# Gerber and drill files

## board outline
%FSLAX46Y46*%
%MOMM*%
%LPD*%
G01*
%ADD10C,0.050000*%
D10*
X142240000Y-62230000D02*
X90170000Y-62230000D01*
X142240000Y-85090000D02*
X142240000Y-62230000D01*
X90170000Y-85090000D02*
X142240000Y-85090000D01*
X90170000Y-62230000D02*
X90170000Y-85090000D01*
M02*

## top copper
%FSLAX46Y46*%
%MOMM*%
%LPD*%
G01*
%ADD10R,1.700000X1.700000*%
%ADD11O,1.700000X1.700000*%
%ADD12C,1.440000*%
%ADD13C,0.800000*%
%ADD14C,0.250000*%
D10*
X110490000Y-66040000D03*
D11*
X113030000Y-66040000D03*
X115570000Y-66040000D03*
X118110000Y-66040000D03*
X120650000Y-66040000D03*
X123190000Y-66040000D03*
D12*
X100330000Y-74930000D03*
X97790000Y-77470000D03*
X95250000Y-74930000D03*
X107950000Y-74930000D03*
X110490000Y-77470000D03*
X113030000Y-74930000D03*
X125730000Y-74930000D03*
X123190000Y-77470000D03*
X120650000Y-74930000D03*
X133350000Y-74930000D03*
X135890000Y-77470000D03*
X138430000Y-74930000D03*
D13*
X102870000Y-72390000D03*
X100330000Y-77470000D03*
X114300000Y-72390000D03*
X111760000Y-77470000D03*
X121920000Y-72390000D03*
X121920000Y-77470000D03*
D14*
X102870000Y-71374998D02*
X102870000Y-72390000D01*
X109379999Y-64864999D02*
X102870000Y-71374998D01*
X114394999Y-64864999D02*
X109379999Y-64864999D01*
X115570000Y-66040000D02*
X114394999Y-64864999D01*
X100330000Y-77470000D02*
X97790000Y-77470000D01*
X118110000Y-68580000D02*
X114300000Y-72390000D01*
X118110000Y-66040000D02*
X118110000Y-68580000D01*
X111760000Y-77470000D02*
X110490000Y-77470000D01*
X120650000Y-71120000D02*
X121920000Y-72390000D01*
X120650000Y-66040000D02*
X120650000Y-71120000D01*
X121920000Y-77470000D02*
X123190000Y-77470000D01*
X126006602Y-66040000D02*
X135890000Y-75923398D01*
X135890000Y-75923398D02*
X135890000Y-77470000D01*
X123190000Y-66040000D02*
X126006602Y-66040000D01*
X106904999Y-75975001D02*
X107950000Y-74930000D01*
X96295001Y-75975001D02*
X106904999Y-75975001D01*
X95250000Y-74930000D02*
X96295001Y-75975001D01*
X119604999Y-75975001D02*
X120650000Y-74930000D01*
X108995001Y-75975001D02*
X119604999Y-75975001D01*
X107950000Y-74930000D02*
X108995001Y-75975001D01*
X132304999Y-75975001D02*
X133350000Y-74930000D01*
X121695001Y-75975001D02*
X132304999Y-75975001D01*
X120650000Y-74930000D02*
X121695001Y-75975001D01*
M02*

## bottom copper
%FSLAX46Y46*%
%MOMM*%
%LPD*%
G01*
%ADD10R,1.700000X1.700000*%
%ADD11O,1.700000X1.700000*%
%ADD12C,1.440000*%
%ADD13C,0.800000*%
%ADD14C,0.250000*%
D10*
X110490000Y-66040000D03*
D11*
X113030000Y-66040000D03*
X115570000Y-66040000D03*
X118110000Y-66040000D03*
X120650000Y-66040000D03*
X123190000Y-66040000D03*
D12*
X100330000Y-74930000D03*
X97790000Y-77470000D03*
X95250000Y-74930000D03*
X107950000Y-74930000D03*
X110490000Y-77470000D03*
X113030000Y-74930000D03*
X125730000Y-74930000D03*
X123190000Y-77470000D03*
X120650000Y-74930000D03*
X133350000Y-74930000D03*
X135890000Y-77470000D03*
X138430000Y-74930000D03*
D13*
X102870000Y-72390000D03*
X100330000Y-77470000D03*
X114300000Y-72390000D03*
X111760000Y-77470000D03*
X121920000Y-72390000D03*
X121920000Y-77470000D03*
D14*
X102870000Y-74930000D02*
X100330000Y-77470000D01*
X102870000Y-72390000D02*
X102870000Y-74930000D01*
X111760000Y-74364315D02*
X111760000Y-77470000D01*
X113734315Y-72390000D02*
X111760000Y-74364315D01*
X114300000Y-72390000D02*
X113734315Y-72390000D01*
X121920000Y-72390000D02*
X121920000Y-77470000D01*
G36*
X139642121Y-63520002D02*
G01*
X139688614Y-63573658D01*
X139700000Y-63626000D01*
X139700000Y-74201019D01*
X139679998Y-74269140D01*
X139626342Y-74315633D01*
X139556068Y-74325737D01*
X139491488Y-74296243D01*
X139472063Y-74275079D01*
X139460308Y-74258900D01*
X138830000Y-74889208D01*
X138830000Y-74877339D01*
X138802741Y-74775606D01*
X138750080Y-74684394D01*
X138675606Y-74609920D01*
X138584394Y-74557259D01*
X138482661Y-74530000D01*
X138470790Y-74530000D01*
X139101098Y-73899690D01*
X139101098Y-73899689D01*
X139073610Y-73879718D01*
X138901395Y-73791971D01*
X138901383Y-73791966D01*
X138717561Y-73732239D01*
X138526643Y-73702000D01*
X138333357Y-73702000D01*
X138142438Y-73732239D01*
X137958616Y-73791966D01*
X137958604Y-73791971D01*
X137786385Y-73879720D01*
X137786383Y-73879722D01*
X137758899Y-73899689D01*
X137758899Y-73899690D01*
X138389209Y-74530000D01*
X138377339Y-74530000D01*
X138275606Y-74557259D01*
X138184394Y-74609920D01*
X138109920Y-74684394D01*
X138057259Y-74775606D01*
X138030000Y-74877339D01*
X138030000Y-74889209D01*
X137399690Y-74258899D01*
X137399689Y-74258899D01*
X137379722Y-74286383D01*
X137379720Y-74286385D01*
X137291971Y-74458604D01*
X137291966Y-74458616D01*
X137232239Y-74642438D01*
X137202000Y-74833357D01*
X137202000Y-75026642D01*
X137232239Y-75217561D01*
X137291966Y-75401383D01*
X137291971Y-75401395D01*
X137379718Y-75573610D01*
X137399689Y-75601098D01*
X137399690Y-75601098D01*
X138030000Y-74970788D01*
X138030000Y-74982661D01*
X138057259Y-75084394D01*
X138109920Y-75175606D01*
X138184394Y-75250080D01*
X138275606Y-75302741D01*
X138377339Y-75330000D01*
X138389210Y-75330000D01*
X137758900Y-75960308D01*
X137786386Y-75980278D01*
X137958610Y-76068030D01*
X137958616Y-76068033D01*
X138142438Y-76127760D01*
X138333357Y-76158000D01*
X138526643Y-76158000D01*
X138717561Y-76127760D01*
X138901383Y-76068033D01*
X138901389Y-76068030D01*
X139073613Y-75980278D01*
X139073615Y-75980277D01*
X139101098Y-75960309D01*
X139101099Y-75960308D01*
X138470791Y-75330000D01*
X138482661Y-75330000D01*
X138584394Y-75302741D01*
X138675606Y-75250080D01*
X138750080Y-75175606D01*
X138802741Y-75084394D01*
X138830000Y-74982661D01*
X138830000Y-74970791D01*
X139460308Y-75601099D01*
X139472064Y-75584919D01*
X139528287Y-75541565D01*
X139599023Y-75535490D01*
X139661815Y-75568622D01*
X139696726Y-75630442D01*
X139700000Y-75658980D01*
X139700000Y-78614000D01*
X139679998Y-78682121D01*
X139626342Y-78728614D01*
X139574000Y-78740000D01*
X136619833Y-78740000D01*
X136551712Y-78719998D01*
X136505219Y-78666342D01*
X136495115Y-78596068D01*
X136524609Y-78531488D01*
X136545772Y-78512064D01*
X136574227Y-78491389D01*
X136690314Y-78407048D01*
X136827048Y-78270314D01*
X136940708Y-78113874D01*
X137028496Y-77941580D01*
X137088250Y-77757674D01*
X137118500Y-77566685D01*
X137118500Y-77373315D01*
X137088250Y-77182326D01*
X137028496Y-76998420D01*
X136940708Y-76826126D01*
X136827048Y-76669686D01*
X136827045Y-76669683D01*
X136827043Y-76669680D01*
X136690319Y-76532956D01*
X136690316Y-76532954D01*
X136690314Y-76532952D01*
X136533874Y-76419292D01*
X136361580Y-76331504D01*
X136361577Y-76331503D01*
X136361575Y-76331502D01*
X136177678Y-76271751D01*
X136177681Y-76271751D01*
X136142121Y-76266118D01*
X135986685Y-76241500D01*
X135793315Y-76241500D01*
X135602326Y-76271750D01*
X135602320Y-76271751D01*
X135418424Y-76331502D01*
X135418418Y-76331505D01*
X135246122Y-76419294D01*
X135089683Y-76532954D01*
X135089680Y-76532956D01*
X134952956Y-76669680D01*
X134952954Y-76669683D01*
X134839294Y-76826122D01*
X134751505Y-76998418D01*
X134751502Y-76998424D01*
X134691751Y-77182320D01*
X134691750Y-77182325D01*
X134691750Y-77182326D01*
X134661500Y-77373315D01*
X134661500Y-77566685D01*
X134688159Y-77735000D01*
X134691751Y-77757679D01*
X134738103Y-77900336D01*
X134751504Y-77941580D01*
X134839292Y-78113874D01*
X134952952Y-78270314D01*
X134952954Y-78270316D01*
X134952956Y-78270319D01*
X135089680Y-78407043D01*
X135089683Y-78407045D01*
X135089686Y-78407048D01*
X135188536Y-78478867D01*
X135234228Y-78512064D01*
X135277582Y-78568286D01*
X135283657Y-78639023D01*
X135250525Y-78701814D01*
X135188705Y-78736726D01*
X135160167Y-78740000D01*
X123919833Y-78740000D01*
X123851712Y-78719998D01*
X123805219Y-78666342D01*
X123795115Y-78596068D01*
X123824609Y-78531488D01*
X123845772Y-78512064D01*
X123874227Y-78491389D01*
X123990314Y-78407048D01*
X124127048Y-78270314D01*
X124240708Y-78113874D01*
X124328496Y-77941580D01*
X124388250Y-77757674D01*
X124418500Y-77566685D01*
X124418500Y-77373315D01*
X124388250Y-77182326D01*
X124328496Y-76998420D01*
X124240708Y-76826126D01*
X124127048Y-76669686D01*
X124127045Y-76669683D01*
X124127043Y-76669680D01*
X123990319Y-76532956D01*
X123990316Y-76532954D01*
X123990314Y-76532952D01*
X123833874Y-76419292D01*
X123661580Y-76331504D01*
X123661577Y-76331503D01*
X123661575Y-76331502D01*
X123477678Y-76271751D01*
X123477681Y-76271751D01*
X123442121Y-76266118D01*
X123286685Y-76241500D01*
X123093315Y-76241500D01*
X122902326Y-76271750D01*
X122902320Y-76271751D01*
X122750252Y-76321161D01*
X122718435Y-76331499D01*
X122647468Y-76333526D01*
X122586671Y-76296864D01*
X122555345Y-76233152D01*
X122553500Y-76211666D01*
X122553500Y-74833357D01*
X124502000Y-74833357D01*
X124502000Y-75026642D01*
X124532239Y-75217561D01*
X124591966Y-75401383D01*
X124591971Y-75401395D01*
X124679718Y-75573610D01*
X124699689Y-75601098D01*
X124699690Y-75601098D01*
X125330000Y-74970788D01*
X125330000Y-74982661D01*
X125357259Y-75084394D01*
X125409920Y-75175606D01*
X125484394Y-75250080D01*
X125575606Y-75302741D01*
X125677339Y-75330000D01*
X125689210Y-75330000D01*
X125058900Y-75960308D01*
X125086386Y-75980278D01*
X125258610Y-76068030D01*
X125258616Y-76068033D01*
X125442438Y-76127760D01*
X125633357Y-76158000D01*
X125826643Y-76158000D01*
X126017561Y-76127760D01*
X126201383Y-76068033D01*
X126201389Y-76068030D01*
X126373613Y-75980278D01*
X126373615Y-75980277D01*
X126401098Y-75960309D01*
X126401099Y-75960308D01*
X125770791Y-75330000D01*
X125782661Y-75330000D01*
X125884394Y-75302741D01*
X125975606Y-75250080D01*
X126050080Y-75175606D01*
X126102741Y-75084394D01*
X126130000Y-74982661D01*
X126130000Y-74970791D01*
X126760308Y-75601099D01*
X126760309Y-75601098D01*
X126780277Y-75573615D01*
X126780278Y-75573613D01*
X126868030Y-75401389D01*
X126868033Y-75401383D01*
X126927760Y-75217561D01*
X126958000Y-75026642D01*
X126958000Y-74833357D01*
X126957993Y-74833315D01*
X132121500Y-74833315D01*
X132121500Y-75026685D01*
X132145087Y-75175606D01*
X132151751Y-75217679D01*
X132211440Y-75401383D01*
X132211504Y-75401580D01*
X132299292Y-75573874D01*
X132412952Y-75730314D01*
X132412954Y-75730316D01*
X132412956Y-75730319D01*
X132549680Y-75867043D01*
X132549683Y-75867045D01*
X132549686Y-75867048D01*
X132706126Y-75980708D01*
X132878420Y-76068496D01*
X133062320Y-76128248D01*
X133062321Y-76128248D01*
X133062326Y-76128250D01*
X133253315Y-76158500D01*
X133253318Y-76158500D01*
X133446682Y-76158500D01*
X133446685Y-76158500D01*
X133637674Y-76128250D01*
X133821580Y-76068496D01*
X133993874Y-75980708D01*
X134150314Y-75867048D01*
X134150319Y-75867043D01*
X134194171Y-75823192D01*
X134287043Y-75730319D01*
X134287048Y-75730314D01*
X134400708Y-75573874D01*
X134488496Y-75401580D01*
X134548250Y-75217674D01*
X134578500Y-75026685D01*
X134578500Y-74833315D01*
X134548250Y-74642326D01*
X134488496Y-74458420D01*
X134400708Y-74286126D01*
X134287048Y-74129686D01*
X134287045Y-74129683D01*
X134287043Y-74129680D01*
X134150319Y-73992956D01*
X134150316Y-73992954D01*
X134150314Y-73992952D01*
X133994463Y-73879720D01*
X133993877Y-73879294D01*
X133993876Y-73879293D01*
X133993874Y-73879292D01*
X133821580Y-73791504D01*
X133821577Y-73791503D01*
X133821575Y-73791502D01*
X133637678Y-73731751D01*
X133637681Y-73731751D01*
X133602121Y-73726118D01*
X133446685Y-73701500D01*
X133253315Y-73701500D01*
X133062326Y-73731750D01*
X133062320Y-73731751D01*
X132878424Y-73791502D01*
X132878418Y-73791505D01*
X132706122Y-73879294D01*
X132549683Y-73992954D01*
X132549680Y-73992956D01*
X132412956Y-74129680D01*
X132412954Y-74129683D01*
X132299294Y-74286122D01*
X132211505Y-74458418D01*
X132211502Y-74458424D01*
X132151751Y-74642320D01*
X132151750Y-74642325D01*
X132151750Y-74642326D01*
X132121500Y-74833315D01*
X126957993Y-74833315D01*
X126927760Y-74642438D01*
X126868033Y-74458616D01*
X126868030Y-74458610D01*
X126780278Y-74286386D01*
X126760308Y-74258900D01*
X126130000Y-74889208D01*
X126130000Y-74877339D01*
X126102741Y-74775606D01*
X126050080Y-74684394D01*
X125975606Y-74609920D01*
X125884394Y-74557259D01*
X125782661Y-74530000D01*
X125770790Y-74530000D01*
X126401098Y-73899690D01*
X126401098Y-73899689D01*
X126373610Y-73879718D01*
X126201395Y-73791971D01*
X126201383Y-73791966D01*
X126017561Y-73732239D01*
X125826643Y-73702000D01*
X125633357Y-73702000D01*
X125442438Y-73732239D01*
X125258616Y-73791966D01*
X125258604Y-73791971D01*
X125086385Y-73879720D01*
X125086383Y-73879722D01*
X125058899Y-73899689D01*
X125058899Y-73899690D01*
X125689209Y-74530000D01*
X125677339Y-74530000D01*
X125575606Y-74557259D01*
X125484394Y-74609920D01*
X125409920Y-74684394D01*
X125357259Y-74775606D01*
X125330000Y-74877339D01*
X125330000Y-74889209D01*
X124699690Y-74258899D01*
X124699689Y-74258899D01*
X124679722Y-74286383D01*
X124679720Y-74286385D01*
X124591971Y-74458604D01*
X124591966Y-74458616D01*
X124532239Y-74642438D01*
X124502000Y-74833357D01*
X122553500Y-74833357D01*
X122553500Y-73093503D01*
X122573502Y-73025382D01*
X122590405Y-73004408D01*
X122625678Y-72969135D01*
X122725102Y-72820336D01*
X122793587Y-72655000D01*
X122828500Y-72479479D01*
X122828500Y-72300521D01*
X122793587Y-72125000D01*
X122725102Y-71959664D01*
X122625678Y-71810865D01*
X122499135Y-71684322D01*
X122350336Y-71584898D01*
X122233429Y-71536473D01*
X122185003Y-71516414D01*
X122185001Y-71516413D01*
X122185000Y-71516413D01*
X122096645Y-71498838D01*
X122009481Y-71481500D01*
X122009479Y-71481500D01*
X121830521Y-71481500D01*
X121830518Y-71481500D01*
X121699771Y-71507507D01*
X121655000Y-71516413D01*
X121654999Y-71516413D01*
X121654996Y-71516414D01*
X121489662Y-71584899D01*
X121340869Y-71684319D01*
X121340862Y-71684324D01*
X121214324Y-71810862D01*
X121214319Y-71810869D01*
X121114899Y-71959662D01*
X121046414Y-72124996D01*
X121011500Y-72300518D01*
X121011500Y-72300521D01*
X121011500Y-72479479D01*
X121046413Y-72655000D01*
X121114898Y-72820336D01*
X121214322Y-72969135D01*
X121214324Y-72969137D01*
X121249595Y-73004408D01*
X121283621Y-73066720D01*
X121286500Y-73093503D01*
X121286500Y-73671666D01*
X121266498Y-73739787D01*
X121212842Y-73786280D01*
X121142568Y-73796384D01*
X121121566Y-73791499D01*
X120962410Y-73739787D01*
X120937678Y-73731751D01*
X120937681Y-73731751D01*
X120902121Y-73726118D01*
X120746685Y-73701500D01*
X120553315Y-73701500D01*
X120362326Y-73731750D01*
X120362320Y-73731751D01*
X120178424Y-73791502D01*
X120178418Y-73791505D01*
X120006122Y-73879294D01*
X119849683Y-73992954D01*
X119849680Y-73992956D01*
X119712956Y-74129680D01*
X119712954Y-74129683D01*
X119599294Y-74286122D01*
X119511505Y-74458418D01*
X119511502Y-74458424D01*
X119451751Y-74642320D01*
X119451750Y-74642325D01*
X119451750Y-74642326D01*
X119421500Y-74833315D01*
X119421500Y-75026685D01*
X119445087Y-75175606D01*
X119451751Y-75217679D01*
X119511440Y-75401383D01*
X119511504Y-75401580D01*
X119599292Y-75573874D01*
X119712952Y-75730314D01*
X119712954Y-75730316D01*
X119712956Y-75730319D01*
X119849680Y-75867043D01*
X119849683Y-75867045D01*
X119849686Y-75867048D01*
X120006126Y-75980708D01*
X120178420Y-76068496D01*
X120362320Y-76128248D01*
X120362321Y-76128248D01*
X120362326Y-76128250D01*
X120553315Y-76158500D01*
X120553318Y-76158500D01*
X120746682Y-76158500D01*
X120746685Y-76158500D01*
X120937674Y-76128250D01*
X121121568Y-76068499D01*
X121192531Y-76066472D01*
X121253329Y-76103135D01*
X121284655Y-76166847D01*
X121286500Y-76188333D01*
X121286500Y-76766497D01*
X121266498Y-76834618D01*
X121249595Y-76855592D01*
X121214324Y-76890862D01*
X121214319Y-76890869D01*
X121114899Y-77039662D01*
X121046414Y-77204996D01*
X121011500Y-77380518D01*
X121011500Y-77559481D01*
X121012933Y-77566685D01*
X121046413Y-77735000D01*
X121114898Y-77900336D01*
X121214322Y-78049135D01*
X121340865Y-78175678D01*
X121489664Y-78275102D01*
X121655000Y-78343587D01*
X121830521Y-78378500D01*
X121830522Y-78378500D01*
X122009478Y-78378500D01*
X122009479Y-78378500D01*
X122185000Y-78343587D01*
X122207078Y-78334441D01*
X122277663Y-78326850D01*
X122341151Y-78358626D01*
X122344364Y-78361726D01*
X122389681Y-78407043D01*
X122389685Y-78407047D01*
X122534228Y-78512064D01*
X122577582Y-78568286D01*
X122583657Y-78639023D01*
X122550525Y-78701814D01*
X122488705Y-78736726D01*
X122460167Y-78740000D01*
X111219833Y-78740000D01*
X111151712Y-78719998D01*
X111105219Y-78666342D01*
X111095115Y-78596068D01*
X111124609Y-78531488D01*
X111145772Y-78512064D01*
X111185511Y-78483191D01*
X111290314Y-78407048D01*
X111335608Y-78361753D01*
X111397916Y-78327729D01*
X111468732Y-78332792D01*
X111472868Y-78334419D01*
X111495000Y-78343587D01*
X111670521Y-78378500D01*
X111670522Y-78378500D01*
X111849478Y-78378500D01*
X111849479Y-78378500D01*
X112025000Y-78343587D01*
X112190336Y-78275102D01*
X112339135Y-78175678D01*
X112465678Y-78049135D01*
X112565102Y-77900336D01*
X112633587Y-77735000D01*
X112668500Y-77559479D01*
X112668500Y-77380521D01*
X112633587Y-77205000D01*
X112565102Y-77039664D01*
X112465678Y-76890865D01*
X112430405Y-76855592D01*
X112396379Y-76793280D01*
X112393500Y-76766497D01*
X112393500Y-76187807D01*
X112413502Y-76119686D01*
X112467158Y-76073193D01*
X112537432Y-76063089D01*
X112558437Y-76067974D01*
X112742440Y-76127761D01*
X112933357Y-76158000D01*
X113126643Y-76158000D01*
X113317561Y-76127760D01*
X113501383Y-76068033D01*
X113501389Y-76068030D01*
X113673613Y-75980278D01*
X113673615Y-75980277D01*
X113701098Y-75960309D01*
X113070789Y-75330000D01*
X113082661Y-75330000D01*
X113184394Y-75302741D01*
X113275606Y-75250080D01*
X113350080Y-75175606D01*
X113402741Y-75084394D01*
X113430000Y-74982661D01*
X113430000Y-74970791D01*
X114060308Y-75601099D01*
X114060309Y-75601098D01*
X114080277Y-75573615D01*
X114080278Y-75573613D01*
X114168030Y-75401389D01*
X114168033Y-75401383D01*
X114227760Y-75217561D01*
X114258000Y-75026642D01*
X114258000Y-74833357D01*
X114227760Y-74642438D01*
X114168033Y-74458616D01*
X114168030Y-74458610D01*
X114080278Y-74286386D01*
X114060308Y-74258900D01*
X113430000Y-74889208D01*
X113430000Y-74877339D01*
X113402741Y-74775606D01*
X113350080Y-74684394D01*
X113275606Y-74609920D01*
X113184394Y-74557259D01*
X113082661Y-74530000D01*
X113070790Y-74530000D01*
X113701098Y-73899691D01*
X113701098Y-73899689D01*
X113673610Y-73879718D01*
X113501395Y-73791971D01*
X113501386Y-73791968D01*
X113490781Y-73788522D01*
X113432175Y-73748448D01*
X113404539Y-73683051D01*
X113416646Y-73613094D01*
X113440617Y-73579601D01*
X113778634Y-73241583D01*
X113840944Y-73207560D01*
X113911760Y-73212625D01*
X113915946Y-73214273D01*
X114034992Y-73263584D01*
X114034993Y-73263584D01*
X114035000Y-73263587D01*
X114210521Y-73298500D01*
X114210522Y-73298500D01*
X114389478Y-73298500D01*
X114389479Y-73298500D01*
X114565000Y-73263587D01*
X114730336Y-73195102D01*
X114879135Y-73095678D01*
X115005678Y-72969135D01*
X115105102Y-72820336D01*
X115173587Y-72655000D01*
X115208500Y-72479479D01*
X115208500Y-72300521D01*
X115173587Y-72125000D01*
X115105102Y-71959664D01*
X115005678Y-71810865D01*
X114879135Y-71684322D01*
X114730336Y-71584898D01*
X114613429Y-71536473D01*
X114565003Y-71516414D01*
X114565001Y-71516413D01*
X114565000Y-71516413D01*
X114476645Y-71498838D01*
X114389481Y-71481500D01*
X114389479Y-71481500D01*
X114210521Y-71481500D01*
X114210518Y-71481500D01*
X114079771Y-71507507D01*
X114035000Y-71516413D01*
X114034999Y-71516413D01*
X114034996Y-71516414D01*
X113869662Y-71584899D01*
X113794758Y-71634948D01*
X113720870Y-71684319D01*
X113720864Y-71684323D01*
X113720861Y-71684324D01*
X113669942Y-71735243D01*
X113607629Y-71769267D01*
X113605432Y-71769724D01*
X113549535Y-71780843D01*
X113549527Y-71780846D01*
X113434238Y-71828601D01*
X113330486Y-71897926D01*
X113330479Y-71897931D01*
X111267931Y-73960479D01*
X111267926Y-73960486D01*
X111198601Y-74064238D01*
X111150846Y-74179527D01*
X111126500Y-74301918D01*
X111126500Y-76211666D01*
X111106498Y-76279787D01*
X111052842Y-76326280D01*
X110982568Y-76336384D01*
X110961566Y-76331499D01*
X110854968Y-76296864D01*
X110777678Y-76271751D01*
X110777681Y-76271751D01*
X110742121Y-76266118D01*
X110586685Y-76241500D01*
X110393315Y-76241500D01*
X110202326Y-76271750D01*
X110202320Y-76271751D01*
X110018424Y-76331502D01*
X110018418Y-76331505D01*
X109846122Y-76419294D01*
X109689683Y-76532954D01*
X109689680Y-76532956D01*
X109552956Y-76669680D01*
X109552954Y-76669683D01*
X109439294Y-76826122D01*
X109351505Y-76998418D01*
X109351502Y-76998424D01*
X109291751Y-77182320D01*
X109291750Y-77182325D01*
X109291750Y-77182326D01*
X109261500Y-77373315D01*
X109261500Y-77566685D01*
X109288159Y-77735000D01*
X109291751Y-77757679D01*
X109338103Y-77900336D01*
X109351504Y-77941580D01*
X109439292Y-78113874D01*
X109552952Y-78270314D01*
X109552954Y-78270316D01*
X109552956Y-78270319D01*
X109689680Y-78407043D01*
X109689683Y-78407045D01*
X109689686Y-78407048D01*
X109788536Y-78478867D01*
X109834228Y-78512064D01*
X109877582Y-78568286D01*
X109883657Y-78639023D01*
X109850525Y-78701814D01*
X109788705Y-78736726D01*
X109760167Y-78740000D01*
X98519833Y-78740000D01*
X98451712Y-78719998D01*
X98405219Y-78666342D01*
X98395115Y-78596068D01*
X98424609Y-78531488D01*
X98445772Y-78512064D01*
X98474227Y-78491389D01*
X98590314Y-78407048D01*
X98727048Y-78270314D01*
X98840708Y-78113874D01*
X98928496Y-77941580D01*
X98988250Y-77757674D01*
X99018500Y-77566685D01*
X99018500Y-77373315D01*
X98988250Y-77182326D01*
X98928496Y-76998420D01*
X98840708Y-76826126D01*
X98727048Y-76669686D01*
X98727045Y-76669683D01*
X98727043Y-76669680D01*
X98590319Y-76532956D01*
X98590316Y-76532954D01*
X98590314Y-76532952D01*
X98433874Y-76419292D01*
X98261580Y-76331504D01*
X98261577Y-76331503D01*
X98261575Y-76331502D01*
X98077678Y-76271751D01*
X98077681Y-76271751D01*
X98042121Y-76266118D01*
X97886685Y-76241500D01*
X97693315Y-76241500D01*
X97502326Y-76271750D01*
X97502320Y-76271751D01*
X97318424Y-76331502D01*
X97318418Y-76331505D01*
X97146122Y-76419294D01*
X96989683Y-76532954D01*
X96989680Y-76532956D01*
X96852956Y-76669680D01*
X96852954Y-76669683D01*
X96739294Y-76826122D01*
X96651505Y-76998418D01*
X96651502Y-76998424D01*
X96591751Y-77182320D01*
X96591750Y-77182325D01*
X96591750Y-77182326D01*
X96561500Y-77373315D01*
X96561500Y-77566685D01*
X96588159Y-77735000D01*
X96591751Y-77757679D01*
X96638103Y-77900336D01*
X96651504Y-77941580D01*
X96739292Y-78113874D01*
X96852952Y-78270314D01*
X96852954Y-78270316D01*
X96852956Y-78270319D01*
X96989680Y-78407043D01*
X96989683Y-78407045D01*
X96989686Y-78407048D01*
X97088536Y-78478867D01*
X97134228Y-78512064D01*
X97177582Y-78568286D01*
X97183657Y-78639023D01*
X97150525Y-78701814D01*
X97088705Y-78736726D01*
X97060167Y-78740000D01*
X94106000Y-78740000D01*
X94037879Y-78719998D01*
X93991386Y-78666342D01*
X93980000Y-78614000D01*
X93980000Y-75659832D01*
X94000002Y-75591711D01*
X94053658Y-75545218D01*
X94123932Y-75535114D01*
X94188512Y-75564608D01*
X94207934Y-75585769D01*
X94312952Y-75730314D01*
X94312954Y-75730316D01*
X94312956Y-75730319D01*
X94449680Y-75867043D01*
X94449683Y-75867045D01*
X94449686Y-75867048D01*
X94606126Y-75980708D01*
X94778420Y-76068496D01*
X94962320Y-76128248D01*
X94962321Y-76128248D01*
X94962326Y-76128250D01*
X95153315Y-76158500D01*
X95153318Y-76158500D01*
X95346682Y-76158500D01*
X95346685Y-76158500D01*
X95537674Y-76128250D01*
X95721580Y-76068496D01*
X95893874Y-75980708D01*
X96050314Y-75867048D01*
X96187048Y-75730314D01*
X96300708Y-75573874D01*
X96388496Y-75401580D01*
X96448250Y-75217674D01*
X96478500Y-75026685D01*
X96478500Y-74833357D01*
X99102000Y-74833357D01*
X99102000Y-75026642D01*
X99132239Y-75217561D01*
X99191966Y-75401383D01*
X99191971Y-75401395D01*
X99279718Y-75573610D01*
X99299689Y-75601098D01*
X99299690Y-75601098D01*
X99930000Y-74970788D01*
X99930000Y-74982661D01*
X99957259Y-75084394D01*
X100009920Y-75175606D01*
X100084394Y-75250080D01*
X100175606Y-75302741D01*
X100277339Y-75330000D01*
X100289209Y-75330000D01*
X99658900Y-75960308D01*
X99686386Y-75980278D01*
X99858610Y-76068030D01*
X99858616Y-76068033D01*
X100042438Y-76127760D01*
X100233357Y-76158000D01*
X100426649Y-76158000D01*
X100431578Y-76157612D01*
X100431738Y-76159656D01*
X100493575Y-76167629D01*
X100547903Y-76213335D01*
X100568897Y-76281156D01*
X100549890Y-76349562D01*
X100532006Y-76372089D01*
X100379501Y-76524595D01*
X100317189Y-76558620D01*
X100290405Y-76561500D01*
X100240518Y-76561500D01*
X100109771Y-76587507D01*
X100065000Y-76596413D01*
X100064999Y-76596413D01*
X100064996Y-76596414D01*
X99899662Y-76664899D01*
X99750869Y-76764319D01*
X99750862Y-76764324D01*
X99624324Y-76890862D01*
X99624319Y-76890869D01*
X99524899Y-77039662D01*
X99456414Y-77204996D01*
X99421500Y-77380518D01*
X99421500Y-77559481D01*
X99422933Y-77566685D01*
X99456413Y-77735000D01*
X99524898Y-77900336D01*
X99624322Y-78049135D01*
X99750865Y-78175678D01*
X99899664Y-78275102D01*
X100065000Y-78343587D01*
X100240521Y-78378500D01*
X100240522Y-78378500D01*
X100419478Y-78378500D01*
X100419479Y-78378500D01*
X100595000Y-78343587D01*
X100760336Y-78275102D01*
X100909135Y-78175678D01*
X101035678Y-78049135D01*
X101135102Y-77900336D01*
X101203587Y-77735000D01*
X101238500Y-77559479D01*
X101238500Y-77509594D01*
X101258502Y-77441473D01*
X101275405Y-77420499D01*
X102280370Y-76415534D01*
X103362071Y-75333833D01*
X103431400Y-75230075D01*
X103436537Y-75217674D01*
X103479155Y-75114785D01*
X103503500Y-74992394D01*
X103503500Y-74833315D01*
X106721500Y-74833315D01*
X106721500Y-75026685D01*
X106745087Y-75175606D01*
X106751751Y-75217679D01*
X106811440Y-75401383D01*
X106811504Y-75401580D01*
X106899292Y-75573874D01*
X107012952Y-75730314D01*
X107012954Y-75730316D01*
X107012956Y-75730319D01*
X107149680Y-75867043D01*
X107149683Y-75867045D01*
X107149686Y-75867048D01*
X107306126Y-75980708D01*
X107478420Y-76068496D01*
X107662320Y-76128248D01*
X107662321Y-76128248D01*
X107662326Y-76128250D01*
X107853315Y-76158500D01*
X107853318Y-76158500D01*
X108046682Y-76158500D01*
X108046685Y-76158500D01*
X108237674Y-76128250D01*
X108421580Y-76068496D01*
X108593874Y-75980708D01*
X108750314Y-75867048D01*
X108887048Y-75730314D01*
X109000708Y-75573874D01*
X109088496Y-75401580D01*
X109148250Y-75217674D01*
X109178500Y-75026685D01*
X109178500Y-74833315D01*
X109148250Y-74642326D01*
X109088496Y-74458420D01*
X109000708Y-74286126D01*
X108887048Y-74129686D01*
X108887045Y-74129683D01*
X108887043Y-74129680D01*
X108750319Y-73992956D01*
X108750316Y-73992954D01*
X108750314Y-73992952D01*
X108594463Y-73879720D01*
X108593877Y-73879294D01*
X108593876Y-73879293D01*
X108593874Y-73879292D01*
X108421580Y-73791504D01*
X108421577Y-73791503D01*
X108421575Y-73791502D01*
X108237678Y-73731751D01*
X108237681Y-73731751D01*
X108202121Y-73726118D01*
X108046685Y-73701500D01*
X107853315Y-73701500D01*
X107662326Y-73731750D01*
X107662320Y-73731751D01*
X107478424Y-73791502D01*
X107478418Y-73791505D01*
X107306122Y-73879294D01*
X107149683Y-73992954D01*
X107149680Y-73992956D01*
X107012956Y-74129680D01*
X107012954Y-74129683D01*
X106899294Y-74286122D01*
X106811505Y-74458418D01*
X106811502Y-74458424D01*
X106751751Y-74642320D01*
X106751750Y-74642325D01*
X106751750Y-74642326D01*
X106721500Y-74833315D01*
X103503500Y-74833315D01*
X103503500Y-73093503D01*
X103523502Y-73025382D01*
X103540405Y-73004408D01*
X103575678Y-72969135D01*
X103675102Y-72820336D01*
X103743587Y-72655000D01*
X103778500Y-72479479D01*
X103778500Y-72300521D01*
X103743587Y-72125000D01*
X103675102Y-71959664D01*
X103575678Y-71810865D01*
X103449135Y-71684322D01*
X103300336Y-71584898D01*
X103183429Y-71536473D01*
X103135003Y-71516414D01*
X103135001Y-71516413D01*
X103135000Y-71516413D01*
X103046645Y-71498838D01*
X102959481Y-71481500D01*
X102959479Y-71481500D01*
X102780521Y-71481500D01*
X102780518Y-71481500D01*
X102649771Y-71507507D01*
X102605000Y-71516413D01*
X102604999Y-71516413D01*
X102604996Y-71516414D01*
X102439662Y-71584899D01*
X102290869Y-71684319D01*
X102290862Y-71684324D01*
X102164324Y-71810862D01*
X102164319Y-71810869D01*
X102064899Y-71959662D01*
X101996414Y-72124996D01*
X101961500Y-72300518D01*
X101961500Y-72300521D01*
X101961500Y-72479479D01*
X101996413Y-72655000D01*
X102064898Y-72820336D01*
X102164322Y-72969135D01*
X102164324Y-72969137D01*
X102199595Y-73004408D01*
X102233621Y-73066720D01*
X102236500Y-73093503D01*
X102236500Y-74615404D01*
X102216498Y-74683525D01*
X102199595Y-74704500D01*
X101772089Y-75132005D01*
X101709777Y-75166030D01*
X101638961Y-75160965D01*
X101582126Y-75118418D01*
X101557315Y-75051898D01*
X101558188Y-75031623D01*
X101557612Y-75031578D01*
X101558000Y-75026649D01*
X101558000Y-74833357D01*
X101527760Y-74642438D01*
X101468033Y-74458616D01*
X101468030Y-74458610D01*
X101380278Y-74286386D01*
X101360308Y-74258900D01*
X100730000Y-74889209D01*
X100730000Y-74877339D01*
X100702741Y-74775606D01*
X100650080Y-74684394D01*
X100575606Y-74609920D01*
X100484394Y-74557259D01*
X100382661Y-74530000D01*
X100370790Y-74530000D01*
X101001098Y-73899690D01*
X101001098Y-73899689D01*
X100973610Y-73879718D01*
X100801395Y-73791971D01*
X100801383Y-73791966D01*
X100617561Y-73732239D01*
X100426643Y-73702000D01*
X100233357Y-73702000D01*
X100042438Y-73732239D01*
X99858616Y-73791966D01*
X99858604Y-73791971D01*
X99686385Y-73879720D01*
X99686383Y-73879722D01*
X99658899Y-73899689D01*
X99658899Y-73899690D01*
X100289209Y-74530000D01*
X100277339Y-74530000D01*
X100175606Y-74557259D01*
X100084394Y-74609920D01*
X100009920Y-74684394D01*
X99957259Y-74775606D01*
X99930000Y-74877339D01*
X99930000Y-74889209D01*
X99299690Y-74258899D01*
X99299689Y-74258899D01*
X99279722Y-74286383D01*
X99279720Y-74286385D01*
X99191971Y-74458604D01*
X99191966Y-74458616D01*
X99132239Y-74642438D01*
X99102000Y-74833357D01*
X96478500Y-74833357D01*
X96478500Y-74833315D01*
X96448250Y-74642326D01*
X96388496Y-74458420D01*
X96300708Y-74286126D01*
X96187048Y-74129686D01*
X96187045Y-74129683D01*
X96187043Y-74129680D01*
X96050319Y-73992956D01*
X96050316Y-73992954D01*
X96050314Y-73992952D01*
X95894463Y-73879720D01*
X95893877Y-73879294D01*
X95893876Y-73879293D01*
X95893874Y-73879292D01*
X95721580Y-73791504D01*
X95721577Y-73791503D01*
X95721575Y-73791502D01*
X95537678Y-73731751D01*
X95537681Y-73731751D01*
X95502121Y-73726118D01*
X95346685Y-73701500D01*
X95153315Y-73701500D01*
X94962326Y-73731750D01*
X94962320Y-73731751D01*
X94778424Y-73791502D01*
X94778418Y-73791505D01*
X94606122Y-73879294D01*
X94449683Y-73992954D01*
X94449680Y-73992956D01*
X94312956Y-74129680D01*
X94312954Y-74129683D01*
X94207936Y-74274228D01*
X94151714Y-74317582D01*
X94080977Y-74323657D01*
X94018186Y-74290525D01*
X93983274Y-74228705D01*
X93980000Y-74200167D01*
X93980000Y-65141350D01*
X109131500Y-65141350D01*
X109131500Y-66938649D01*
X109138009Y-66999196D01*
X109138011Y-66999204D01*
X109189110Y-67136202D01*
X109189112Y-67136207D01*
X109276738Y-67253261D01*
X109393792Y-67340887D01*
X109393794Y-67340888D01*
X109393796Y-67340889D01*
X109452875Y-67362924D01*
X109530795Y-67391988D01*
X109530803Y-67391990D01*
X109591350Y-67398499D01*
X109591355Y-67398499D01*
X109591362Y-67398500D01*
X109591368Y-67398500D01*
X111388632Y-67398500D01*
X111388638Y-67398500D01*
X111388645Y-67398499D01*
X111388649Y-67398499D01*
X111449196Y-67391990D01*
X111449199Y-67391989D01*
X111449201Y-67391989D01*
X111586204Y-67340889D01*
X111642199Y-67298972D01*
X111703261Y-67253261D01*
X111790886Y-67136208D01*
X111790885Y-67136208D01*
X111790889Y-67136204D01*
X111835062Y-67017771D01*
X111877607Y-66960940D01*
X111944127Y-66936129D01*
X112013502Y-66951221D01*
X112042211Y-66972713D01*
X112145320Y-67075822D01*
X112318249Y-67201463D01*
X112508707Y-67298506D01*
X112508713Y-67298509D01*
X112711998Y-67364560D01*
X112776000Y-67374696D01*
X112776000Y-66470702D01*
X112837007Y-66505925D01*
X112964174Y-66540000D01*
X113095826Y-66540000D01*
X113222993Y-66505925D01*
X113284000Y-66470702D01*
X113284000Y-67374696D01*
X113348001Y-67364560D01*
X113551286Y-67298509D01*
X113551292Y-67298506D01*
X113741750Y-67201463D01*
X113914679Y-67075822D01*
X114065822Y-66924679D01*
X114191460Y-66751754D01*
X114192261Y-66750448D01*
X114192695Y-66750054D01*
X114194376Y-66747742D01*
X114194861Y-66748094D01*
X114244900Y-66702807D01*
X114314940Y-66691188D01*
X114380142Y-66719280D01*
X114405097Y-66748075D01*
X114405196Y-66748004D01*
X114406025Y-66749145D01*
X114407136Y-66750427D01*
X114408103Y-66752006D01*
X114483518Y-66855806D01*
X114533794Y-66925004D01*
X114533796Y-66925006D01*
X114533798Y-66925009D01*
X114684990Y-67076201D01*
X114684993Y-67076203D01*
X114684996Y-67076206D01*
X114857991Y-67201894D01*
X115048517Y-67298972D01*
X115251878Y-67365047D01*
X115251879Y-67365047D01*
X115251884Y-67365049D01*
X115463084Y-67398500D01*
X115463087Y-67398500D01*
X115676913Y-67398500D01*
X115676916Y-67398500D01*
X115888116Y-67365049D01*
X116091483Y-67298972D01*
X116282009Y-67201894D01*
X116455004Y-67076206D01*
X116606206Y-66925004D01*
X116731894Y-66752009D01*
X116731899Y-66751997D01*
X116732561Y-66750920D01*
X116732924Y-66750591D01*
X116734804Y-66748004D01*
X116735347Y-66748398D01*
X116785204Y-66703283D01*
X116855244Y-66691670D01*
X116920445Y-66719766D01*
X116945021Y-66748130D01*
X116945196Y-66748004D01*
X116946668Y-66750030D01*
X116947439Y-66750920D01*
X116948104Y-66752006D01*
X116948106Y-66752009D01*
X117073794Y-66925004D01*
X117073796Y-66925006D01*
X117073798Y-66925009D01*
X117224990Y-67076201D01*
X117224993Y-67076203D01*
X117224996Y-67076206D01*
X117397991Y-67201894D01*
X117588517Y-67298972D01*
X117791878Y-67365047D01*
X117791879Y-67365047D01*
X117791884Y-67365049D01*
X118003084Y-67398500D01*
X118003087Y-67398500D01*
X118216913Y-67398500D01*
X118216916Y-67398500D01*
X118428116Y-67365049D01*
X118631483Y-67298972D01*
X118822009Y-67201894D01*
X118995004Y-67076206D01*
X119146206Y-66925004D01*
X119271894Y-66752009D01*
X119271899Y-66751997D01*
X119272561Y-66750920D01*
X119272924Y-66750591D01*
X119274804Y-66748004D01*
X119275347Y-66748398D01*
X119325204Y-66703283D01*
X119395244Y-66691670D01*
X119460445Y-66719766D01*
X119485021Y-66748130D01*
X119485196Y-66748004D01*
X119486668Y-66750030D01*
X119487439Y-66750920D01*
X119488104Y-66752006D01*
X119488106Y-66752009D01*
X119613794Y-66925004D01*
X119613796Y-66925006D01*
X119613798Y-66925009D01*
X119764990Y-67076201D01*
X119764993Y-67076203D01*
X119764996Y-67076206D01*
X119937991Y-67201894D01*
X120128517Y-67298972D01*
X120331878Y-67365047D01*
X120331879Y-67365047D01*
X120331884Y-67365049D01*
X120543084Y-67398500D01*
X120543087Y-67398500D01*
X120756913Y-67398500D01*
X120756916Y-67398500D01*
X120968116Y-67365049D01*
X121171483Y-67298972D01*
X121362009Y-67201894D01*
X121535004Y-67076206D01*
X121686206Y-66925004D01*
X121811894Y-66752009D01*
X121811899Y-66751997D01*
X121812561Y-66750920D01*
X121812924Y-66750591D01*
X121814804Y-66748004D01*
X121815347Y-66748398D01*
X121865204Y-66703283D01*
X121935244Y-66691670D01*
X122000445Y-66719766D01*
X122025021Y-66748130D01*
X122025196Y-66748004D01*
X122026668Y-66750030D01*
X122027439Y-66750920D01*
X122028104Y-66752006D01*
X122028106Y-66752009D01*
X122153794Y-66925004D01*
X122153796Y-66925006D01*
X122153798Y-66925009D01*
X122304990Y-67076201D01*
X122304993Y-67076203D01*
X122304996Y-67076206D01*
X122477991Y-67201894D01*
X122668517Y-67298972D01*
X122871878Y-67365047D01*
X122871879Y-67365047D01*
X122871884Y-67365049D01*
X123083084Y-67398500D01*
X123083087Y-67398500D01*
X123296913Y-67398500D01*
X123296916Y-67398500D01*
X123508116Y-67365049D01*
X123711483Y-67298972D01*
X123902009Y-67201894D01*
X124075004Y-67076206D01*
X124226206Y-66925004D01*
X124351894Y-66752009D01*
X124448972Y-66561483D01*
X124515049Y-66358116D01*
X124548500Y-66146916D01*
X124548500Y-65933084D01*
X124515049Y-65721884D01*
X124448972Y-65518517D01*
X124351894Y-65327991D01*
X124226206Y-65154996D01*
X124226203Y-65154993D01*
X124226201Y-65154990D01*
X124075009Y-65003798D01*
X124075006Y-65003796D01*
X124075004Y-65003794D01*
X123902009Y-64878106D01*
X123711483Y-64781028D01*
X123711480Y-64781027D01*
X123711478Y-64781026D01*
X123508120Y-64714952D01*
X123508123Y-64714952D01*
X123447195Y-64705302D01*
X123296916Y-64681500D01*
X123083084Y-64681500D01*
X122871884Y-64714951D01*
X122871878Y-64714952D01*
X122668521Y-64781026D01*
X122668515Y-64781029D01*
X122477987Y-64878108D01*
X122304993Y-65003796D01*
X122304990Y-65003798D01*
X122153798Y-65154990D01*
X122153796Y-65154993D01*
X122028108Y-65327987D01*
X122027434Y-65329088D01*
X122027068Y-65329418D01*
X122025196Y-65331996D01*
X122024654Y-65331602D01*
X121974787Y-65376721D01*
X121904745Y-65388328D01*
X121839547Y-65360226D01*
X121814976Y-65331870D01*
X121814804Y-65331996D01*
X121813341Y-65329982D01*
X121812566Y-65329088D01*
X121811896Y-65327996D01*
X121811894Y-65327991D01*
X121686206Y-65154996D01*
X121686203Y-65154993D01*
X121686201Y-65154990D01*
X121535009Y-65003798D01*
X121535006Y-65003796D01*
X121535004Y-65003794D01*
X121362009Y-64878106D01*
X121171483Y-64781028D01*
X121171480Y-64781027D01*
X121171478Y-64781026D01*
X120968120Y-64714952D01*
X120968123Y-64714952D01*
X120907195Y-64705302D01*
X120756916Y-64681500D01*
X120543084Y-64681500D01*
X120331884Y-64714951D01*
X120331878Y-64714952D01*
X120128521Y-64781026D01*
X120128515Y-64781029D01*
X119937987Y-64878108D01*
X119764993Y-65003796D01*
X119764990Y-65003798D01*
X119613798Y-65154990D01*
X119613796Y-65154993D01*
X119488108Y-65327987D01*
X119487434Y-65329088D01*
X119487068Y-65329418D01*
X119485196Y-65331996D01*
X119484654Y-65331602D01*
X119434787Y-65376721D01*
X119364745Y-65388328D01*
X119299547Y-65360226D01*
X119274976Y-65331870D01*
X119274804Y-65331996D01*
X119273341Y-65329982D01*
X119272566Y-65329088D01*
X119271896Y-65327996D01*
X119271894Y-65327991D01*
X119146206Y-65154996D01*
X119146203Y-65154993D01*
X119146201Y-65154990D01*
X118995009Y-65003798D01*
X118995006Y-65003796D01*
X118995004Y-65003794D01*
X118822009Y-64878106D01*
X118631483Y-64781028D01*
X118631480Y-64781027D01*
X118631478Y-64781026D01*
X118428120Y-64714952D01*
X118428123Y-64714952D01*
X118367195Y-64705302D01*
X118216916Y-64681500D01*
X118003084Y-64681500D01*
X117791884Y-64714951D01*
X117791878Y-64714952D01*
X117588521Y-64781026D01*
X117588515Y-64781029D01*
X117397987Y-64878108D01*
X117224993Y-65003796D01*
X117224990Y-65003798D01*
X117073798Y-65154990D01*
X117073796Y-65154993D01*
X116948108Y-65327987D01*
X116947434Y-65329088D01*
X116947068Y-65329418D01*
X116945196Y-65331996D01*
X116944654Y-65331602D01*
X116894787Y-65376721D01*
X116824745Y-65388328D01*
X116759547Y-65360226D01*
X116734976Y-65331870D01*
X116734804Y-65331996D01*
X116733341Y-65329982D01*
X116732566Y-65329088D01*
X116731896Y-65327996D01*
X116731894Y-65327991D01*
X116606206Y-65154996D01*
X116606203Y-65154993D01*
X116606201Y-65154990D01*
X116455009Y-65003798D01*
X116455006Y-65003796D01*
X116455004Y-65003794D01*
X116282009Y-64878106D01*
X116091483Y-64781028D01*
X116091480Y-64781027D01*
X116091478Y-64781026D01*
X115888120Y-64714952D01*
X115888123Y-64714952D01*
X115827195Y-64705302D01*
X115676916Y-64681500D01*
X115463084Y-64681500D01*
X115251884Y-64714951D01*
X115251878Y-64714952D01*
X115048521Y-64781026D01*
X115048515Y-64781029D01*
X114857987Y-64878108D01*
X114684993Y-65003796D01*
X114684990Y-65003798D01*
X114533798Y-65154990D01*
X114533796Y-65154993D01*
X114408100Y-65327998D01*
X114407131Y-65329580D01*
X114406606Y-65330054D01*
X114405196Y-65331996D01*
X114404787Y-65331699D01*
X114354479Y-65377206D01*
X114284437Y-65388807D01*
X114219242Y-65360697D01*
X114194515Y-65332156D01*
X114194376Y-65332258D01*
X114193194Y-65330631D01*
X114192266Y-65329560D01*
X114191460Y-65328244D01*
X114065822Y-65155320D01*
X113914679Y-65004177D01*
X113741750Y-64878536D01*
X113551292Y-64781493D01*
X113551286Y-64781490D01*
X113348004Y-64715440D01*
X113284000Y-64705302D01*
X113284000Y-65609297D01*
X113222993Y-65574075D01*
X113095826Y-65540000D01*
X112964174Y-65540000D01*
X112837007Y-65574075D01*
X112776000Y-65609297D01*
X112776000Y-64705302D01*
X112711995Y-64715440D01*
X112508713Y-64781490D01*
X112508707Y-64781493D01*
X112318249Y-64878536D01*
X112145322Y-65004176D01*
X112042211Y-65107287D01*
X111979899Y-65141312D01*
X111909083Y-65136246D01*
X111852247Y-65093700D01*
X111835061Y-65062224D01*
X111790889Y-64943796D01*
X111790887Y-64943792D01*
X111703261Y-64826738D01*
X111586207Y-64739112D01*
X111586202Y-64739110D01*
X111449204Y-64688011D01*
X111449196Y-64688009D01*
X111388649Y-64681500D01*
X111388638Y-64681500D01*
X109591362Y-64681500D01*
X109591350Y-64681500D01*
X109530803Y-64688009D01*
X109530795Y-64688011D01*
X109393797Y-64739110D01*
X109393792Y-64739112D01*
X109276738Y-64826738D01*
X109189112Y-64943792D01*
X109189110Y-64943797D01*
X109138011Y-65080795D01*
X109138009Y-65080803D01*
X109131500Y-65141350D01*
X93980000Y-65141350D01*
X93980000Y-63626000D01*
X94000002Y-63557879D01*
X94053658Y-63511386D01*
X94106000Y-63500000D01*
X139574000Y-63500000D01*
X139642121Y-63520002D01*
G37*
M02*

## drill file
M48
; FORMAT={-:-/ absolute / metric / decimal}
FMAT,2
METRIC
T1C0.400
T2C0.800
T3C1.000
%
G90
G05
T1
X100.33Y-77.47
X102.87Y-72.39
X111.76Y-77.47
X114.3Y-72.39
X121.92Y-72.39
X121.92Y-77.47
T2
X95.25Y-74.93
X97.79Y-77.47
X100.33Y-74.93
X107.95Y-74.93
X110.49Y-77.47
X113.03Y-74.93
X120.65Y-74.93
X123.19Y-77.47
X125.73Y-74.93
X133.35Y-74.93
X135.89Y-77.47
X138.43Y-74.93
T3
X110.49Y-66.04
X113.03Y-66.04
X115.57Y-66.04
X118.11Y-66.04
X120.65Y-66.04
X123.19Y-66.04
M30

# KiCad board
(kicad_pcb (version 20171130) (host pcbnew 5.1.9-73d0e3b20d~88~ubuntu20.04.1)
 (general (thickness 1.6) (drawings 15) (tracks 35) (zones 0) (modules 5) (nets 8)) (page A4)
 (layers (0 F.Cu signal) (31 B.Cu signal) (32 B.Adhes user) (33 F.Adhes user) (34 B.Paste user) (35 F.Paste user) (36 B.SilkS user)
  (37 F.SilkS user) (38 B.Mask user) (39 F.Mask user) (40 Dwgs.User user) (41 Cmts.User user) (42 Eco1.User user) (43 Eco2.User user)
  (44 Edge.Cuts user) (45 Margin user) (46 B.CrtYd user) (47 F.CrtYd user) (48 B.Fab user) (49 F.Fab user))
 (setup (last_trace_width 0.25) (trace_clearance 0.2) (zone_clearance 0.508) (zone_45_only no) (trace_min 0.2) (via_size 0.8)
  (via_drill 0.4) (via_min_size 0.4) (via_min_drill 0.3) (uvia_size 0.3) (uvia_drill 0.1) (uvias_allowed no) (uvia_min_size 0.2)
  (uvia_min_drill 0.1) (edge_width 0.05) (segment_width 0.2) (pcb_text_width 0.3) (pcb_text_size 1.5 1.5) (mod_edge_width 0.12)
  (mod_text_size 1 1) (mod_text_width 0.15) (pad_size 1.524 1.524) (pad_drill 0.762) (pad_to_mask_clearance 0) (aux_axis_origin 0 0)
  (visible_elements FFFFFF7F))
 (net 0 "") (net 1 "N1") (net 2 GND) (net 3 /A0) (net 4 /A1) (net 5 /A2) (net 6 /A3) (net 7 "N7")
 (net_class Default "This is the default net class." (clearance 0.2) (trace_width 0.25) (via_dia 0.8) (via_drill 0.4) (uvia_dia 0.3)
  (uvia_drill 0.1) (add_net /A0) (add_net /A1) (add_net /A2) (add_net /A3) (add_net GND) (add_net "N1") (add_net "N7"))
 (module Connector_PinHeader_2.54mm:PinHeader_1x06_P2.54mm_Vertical (layer F.Cu) (at 110.49 66.04 90)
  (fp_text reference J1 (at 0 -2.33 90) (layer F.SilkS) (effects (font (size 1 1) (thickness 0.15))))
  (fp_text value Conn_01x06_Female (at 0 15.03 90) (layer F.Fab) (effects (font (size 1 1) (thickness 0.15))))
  (pad 1 thru_hole rect (at 0 0 90) (size 1.7 1.7) (drill 1) (layers *.Cu *.Mask) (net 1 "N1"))
  (pad 2 thru_hole oval (at 0 2.54 90) (size 1.7 1.7) (drill 1) (layers *.Cu *.Mask) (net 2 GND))
  (pad 3 thru_hole oval (at 0 5.08 90) (size 1.7 1.7) (drill 1) (layers *.Cu *.Mask) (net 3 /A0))
  (pad 4 thru_hole oval (at 0 7.62 90) (size 1.7 1.7) (drill 1) (layers *.Cu *.Mask) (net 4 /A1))
  (pad 5 thru_hole oval (at 0 10.16 90) (size 1.7 1.7) (drill 1) (layers *.Cu *.Mask) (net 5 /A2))
  (pad 6 thru_hole oval (at 0 12.7 90) (size 1.7 1.7) (drill 1) (layers *.Cu *.Mask) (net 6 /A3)))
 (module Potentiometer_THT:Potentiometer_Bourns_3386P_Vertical (layer F.Cu) (at 95.25 74.93 270)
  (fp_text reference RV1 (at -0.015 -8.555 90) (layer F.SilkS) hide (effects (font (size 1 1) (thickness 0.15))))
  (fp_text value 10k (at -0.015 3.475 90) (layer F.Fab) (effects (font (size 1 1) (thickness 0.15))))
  (pad 3 thru_hole circle (at 0 -5.08 270) (size 1.44 1.44) (drill 0.8) (layers *.Cu *.Mask) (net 2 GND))
  (pad 2 thru_hole circle (at 2.54 -2.54 270) (size 1.44 1.44) (drill 0.8) (layers *.Cu *.Mask) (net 3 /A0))
  (pad 1 thru_hole circle (at 0 0 270) (size 1.44 1.44) (drill 0.8) (layers *.Cu *.Mask) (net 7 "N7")))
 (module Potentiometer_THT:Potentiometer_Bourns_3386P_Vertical (layer F.Cu) (at 107.95 74.93 270)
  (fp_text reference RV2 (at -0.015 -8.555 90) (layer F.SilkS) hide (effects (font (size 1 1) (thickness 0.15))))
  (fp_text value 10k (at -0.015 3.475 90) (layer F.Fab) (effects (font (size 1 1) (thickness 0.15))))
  (pad 1 thru_hole circle (at 0 0 270) (size 1.44 1.44) (drill 0.8) (layers *.Cu *.Mask) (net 7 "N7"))
  (pad 2 thru_hole circle (at 2.54 -2.54 270) (size 1.44 1.44) (drill 0.8) (layers *.Cu *.Mask) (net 4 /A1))
  (pad 3 thru_hole circle (at 0 -5.08 270) (size 1.44 1.44) (drill 0.8) (layers *.Cu *.Mask) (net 2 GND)))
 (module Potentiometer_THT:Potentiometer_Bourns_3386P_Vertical (layer F.Cu) (at 120.65 74.93 270)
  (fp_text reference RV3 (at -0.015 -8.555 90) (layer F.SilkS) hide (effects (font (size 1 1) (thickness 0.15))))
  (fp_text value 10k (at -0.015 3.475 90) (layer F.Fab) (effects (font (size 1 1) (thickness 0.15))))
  (pad 3 thru_hole circle (at 0 -5.08 270) (size 1.44 1.44) (drill 0.8) (layers *.Cu *.Mask) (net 2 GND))
  (pad 2 thru_hole circle (at 2.54 -2.54 270) (size 1.44 1.44) (drill 0.8) (layers *.Cu *.Mask) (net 5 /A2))
  (pad 1 thru_hole circle (at 0 0 270) (size 1.44 1.44) (drill 0.8) (layers *.Cu *.Mask) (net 7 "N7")))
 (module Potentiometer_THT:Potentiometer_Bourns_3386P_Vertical (layer F.Cu) (at 133.35 74.93 270)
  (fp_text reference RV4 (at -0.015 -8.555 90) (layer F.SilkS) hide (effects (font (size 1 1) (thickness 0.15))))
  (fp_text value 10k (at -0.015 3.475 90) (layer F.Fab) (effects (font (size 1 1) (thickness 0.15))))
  (pad 1 thru_hole circle (at 0 0 270) (size 1.44 1.44) (drill 0.8) (layers *.Cu *.Mask) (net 7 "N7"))
  (pad 2 thru_hole circle (at 2.54 -2.54 270) (size 1.44 1.44) (drill 0.8) (layers *.Cu *.Mask) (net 6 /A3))
  (pad 3 thru_hole circle (at 0 -5.08 270) (size 1.44 1.44) (drill 0.8) (layers *.Cu *.Mask) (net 2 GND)))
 (gr_line (start 142.24 62.23) (end 90.17 62.23) (layer Edge.Cuts) (width 0.05))
 (gr_line (start 142.24 85.09) (end 142.24 62.23) (layer Edge.Cuts) (width 0.05))
 (gr_line (start 90.17 85.09) (end 142.24 85.09) (layer Edge.Cuts) (width 0.05))
 (gr_line (start 90.17 62.23) (end 90.17 85.09) (layer Edge.Cuts) (width 0.05))
 (via (at 102.87 72.39) (size 0.8) (drill 0.4) (layers F.Cu B.Cu) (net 3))
 (segment (start 102.87 71.374998) (end 102.87 72.39) (width 0.25) (layer F.Cu) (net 3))
 (segment (start 109.379999 64.864999) (end 102.87 71.374998) (width 0.25) (layer F.Cu) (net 3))
 (segment (start 114.394999 64.864999) (end 109.379999 64.864999) (width 0.25) (layer F.Cu) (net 3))
 (segment (start 115.57 66.04) (end 114.394999 64.864999) (width 0.25) (layer F.Cu) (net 3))
 (via (at 100.33 77.47) (size 0.8) (drill 0.4) (layers F.Cu B.Cu) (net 3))
 (segment (start 102.87 74.93) (end 100.33 77.47) (width 0.25) (layer B.Cu) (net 3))
 (segment (start 102.87 72.39) (end 102.87 74.93) (width 0.25) (layer B.Cu) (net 3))
 (segment (start 100.33 77.47) (end 97.79 77.47) (width 0.25) (layer F.Cu) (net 3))
 (via (at 114.3 72.39) (size 0.8) (drill 0.4) (layers F.Cu B.Cu) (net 4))
 (segment (start 118.11 68.58) (end 114.3 72.39) (width 0.25) (layer F.Cu) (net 4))
 (segment (start 118.11 66.04) (end 118.11 68.58) (width 0.25) (layer F.Cu) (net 4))
 (via (at 111.76 77.47) (size 0.8) (drill 0.4) (layers F.Cu B.Cu) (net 4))
 (segment (start 111.76 74.364315) (end 111.76 77.47) (width 0.25) (layer B.Cu) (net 4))
 (segment (start 113.734315 72.39) (end 111.76 74.364315) (width 0.25) (layer B.Cu) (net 4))
 (segment (start 114.3 72.39) (end 113.734315 72.39) (width 0.25) (layer B.Cu) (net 4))
 (segment (start 111.76 77.47) (end 110.49 77.47) (width 0.25) (layer F.Cu) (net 4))
 (via (at 121.92 72.39) (size 0.8) (drill 0.4) (layers F.Cu B.Cu) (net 5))
 (segment (start 120.65 71.12) (end 121.92 72.39) (width 0.25) (layer F.Cu) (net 5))
 (segment (start 120.65 66.04) (end 120.65 71.12) (width 0.25) (layer F.Cu) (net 5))
 (via (at 121.92 77.47) (size 0.8) (drill 0.4) (layers F.Cu B.Cu) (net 5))
 (segment (start 121.92 72.39) (end 121.92 77.47) (width 0.25) (layer B.Cu) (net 5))
 (segment (start 121.92 77.47) (end 123.19 77.47) (width 0.25) (layer F.Cu) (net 5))
 (segment (start 126.006602 66.04) (end 135.89 75.923398) (width 0.25) (layer F.Cu) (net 6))
 (segment (start 135.89 75.923398) (end 135.89 77.47) (width 0.25) (layer F.Cu) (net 6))
 (segment (start 123.19 66.04) (end 126.006602 66.04) (width 0.25) (layer F.Cu) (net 6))
 (segment (start 106.904999 75.975001) (end 107.95 74.93) (width 0.25) (layer F.Cu) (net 7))
 (segment (start 96.295001 75.975001) (end 106.904999 75.975001) (width 0.25) (layer F.Cu) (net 7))
 (segment (start 95.25 74.93) (end 96.295001 75.975001) (width 0.25) (layer F.Cu) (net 7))
 (segment (start 119.604999 75.975001) (end 120.65 74.93) (width 0.25) (layer F.Cu) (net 7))
 (segment (start 108.995001 75.975001) (end 119.604999 75.975001) (width 0.25) (layer F.Cu) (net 7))
 (segment (start 107.95 74.93) (end 108.995001 75.975001) (width 0.25) (layer F.Cu) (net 7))
 (segment (start 132.304999 75.975001) (end 133.35 74.93) (width 0.25) (layer F.Cu) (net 7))
 (segment (start 121.695001 75.975001) (end 132.304999 75.975001) (width 0.25) (layer F.Cu) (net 7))
 (segment (start 120.65 74.93) (end 121.695001 75.975001) (width 0.25) (layer F.Cu) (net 7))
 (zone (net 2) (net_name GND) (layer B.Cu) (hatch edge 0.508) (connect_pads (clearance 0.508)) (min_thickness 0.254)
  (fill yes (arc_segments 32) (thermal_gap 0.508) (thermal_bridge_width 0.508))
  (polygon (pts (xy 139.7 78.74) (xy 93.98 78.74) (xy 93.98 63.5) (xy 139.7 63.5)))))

